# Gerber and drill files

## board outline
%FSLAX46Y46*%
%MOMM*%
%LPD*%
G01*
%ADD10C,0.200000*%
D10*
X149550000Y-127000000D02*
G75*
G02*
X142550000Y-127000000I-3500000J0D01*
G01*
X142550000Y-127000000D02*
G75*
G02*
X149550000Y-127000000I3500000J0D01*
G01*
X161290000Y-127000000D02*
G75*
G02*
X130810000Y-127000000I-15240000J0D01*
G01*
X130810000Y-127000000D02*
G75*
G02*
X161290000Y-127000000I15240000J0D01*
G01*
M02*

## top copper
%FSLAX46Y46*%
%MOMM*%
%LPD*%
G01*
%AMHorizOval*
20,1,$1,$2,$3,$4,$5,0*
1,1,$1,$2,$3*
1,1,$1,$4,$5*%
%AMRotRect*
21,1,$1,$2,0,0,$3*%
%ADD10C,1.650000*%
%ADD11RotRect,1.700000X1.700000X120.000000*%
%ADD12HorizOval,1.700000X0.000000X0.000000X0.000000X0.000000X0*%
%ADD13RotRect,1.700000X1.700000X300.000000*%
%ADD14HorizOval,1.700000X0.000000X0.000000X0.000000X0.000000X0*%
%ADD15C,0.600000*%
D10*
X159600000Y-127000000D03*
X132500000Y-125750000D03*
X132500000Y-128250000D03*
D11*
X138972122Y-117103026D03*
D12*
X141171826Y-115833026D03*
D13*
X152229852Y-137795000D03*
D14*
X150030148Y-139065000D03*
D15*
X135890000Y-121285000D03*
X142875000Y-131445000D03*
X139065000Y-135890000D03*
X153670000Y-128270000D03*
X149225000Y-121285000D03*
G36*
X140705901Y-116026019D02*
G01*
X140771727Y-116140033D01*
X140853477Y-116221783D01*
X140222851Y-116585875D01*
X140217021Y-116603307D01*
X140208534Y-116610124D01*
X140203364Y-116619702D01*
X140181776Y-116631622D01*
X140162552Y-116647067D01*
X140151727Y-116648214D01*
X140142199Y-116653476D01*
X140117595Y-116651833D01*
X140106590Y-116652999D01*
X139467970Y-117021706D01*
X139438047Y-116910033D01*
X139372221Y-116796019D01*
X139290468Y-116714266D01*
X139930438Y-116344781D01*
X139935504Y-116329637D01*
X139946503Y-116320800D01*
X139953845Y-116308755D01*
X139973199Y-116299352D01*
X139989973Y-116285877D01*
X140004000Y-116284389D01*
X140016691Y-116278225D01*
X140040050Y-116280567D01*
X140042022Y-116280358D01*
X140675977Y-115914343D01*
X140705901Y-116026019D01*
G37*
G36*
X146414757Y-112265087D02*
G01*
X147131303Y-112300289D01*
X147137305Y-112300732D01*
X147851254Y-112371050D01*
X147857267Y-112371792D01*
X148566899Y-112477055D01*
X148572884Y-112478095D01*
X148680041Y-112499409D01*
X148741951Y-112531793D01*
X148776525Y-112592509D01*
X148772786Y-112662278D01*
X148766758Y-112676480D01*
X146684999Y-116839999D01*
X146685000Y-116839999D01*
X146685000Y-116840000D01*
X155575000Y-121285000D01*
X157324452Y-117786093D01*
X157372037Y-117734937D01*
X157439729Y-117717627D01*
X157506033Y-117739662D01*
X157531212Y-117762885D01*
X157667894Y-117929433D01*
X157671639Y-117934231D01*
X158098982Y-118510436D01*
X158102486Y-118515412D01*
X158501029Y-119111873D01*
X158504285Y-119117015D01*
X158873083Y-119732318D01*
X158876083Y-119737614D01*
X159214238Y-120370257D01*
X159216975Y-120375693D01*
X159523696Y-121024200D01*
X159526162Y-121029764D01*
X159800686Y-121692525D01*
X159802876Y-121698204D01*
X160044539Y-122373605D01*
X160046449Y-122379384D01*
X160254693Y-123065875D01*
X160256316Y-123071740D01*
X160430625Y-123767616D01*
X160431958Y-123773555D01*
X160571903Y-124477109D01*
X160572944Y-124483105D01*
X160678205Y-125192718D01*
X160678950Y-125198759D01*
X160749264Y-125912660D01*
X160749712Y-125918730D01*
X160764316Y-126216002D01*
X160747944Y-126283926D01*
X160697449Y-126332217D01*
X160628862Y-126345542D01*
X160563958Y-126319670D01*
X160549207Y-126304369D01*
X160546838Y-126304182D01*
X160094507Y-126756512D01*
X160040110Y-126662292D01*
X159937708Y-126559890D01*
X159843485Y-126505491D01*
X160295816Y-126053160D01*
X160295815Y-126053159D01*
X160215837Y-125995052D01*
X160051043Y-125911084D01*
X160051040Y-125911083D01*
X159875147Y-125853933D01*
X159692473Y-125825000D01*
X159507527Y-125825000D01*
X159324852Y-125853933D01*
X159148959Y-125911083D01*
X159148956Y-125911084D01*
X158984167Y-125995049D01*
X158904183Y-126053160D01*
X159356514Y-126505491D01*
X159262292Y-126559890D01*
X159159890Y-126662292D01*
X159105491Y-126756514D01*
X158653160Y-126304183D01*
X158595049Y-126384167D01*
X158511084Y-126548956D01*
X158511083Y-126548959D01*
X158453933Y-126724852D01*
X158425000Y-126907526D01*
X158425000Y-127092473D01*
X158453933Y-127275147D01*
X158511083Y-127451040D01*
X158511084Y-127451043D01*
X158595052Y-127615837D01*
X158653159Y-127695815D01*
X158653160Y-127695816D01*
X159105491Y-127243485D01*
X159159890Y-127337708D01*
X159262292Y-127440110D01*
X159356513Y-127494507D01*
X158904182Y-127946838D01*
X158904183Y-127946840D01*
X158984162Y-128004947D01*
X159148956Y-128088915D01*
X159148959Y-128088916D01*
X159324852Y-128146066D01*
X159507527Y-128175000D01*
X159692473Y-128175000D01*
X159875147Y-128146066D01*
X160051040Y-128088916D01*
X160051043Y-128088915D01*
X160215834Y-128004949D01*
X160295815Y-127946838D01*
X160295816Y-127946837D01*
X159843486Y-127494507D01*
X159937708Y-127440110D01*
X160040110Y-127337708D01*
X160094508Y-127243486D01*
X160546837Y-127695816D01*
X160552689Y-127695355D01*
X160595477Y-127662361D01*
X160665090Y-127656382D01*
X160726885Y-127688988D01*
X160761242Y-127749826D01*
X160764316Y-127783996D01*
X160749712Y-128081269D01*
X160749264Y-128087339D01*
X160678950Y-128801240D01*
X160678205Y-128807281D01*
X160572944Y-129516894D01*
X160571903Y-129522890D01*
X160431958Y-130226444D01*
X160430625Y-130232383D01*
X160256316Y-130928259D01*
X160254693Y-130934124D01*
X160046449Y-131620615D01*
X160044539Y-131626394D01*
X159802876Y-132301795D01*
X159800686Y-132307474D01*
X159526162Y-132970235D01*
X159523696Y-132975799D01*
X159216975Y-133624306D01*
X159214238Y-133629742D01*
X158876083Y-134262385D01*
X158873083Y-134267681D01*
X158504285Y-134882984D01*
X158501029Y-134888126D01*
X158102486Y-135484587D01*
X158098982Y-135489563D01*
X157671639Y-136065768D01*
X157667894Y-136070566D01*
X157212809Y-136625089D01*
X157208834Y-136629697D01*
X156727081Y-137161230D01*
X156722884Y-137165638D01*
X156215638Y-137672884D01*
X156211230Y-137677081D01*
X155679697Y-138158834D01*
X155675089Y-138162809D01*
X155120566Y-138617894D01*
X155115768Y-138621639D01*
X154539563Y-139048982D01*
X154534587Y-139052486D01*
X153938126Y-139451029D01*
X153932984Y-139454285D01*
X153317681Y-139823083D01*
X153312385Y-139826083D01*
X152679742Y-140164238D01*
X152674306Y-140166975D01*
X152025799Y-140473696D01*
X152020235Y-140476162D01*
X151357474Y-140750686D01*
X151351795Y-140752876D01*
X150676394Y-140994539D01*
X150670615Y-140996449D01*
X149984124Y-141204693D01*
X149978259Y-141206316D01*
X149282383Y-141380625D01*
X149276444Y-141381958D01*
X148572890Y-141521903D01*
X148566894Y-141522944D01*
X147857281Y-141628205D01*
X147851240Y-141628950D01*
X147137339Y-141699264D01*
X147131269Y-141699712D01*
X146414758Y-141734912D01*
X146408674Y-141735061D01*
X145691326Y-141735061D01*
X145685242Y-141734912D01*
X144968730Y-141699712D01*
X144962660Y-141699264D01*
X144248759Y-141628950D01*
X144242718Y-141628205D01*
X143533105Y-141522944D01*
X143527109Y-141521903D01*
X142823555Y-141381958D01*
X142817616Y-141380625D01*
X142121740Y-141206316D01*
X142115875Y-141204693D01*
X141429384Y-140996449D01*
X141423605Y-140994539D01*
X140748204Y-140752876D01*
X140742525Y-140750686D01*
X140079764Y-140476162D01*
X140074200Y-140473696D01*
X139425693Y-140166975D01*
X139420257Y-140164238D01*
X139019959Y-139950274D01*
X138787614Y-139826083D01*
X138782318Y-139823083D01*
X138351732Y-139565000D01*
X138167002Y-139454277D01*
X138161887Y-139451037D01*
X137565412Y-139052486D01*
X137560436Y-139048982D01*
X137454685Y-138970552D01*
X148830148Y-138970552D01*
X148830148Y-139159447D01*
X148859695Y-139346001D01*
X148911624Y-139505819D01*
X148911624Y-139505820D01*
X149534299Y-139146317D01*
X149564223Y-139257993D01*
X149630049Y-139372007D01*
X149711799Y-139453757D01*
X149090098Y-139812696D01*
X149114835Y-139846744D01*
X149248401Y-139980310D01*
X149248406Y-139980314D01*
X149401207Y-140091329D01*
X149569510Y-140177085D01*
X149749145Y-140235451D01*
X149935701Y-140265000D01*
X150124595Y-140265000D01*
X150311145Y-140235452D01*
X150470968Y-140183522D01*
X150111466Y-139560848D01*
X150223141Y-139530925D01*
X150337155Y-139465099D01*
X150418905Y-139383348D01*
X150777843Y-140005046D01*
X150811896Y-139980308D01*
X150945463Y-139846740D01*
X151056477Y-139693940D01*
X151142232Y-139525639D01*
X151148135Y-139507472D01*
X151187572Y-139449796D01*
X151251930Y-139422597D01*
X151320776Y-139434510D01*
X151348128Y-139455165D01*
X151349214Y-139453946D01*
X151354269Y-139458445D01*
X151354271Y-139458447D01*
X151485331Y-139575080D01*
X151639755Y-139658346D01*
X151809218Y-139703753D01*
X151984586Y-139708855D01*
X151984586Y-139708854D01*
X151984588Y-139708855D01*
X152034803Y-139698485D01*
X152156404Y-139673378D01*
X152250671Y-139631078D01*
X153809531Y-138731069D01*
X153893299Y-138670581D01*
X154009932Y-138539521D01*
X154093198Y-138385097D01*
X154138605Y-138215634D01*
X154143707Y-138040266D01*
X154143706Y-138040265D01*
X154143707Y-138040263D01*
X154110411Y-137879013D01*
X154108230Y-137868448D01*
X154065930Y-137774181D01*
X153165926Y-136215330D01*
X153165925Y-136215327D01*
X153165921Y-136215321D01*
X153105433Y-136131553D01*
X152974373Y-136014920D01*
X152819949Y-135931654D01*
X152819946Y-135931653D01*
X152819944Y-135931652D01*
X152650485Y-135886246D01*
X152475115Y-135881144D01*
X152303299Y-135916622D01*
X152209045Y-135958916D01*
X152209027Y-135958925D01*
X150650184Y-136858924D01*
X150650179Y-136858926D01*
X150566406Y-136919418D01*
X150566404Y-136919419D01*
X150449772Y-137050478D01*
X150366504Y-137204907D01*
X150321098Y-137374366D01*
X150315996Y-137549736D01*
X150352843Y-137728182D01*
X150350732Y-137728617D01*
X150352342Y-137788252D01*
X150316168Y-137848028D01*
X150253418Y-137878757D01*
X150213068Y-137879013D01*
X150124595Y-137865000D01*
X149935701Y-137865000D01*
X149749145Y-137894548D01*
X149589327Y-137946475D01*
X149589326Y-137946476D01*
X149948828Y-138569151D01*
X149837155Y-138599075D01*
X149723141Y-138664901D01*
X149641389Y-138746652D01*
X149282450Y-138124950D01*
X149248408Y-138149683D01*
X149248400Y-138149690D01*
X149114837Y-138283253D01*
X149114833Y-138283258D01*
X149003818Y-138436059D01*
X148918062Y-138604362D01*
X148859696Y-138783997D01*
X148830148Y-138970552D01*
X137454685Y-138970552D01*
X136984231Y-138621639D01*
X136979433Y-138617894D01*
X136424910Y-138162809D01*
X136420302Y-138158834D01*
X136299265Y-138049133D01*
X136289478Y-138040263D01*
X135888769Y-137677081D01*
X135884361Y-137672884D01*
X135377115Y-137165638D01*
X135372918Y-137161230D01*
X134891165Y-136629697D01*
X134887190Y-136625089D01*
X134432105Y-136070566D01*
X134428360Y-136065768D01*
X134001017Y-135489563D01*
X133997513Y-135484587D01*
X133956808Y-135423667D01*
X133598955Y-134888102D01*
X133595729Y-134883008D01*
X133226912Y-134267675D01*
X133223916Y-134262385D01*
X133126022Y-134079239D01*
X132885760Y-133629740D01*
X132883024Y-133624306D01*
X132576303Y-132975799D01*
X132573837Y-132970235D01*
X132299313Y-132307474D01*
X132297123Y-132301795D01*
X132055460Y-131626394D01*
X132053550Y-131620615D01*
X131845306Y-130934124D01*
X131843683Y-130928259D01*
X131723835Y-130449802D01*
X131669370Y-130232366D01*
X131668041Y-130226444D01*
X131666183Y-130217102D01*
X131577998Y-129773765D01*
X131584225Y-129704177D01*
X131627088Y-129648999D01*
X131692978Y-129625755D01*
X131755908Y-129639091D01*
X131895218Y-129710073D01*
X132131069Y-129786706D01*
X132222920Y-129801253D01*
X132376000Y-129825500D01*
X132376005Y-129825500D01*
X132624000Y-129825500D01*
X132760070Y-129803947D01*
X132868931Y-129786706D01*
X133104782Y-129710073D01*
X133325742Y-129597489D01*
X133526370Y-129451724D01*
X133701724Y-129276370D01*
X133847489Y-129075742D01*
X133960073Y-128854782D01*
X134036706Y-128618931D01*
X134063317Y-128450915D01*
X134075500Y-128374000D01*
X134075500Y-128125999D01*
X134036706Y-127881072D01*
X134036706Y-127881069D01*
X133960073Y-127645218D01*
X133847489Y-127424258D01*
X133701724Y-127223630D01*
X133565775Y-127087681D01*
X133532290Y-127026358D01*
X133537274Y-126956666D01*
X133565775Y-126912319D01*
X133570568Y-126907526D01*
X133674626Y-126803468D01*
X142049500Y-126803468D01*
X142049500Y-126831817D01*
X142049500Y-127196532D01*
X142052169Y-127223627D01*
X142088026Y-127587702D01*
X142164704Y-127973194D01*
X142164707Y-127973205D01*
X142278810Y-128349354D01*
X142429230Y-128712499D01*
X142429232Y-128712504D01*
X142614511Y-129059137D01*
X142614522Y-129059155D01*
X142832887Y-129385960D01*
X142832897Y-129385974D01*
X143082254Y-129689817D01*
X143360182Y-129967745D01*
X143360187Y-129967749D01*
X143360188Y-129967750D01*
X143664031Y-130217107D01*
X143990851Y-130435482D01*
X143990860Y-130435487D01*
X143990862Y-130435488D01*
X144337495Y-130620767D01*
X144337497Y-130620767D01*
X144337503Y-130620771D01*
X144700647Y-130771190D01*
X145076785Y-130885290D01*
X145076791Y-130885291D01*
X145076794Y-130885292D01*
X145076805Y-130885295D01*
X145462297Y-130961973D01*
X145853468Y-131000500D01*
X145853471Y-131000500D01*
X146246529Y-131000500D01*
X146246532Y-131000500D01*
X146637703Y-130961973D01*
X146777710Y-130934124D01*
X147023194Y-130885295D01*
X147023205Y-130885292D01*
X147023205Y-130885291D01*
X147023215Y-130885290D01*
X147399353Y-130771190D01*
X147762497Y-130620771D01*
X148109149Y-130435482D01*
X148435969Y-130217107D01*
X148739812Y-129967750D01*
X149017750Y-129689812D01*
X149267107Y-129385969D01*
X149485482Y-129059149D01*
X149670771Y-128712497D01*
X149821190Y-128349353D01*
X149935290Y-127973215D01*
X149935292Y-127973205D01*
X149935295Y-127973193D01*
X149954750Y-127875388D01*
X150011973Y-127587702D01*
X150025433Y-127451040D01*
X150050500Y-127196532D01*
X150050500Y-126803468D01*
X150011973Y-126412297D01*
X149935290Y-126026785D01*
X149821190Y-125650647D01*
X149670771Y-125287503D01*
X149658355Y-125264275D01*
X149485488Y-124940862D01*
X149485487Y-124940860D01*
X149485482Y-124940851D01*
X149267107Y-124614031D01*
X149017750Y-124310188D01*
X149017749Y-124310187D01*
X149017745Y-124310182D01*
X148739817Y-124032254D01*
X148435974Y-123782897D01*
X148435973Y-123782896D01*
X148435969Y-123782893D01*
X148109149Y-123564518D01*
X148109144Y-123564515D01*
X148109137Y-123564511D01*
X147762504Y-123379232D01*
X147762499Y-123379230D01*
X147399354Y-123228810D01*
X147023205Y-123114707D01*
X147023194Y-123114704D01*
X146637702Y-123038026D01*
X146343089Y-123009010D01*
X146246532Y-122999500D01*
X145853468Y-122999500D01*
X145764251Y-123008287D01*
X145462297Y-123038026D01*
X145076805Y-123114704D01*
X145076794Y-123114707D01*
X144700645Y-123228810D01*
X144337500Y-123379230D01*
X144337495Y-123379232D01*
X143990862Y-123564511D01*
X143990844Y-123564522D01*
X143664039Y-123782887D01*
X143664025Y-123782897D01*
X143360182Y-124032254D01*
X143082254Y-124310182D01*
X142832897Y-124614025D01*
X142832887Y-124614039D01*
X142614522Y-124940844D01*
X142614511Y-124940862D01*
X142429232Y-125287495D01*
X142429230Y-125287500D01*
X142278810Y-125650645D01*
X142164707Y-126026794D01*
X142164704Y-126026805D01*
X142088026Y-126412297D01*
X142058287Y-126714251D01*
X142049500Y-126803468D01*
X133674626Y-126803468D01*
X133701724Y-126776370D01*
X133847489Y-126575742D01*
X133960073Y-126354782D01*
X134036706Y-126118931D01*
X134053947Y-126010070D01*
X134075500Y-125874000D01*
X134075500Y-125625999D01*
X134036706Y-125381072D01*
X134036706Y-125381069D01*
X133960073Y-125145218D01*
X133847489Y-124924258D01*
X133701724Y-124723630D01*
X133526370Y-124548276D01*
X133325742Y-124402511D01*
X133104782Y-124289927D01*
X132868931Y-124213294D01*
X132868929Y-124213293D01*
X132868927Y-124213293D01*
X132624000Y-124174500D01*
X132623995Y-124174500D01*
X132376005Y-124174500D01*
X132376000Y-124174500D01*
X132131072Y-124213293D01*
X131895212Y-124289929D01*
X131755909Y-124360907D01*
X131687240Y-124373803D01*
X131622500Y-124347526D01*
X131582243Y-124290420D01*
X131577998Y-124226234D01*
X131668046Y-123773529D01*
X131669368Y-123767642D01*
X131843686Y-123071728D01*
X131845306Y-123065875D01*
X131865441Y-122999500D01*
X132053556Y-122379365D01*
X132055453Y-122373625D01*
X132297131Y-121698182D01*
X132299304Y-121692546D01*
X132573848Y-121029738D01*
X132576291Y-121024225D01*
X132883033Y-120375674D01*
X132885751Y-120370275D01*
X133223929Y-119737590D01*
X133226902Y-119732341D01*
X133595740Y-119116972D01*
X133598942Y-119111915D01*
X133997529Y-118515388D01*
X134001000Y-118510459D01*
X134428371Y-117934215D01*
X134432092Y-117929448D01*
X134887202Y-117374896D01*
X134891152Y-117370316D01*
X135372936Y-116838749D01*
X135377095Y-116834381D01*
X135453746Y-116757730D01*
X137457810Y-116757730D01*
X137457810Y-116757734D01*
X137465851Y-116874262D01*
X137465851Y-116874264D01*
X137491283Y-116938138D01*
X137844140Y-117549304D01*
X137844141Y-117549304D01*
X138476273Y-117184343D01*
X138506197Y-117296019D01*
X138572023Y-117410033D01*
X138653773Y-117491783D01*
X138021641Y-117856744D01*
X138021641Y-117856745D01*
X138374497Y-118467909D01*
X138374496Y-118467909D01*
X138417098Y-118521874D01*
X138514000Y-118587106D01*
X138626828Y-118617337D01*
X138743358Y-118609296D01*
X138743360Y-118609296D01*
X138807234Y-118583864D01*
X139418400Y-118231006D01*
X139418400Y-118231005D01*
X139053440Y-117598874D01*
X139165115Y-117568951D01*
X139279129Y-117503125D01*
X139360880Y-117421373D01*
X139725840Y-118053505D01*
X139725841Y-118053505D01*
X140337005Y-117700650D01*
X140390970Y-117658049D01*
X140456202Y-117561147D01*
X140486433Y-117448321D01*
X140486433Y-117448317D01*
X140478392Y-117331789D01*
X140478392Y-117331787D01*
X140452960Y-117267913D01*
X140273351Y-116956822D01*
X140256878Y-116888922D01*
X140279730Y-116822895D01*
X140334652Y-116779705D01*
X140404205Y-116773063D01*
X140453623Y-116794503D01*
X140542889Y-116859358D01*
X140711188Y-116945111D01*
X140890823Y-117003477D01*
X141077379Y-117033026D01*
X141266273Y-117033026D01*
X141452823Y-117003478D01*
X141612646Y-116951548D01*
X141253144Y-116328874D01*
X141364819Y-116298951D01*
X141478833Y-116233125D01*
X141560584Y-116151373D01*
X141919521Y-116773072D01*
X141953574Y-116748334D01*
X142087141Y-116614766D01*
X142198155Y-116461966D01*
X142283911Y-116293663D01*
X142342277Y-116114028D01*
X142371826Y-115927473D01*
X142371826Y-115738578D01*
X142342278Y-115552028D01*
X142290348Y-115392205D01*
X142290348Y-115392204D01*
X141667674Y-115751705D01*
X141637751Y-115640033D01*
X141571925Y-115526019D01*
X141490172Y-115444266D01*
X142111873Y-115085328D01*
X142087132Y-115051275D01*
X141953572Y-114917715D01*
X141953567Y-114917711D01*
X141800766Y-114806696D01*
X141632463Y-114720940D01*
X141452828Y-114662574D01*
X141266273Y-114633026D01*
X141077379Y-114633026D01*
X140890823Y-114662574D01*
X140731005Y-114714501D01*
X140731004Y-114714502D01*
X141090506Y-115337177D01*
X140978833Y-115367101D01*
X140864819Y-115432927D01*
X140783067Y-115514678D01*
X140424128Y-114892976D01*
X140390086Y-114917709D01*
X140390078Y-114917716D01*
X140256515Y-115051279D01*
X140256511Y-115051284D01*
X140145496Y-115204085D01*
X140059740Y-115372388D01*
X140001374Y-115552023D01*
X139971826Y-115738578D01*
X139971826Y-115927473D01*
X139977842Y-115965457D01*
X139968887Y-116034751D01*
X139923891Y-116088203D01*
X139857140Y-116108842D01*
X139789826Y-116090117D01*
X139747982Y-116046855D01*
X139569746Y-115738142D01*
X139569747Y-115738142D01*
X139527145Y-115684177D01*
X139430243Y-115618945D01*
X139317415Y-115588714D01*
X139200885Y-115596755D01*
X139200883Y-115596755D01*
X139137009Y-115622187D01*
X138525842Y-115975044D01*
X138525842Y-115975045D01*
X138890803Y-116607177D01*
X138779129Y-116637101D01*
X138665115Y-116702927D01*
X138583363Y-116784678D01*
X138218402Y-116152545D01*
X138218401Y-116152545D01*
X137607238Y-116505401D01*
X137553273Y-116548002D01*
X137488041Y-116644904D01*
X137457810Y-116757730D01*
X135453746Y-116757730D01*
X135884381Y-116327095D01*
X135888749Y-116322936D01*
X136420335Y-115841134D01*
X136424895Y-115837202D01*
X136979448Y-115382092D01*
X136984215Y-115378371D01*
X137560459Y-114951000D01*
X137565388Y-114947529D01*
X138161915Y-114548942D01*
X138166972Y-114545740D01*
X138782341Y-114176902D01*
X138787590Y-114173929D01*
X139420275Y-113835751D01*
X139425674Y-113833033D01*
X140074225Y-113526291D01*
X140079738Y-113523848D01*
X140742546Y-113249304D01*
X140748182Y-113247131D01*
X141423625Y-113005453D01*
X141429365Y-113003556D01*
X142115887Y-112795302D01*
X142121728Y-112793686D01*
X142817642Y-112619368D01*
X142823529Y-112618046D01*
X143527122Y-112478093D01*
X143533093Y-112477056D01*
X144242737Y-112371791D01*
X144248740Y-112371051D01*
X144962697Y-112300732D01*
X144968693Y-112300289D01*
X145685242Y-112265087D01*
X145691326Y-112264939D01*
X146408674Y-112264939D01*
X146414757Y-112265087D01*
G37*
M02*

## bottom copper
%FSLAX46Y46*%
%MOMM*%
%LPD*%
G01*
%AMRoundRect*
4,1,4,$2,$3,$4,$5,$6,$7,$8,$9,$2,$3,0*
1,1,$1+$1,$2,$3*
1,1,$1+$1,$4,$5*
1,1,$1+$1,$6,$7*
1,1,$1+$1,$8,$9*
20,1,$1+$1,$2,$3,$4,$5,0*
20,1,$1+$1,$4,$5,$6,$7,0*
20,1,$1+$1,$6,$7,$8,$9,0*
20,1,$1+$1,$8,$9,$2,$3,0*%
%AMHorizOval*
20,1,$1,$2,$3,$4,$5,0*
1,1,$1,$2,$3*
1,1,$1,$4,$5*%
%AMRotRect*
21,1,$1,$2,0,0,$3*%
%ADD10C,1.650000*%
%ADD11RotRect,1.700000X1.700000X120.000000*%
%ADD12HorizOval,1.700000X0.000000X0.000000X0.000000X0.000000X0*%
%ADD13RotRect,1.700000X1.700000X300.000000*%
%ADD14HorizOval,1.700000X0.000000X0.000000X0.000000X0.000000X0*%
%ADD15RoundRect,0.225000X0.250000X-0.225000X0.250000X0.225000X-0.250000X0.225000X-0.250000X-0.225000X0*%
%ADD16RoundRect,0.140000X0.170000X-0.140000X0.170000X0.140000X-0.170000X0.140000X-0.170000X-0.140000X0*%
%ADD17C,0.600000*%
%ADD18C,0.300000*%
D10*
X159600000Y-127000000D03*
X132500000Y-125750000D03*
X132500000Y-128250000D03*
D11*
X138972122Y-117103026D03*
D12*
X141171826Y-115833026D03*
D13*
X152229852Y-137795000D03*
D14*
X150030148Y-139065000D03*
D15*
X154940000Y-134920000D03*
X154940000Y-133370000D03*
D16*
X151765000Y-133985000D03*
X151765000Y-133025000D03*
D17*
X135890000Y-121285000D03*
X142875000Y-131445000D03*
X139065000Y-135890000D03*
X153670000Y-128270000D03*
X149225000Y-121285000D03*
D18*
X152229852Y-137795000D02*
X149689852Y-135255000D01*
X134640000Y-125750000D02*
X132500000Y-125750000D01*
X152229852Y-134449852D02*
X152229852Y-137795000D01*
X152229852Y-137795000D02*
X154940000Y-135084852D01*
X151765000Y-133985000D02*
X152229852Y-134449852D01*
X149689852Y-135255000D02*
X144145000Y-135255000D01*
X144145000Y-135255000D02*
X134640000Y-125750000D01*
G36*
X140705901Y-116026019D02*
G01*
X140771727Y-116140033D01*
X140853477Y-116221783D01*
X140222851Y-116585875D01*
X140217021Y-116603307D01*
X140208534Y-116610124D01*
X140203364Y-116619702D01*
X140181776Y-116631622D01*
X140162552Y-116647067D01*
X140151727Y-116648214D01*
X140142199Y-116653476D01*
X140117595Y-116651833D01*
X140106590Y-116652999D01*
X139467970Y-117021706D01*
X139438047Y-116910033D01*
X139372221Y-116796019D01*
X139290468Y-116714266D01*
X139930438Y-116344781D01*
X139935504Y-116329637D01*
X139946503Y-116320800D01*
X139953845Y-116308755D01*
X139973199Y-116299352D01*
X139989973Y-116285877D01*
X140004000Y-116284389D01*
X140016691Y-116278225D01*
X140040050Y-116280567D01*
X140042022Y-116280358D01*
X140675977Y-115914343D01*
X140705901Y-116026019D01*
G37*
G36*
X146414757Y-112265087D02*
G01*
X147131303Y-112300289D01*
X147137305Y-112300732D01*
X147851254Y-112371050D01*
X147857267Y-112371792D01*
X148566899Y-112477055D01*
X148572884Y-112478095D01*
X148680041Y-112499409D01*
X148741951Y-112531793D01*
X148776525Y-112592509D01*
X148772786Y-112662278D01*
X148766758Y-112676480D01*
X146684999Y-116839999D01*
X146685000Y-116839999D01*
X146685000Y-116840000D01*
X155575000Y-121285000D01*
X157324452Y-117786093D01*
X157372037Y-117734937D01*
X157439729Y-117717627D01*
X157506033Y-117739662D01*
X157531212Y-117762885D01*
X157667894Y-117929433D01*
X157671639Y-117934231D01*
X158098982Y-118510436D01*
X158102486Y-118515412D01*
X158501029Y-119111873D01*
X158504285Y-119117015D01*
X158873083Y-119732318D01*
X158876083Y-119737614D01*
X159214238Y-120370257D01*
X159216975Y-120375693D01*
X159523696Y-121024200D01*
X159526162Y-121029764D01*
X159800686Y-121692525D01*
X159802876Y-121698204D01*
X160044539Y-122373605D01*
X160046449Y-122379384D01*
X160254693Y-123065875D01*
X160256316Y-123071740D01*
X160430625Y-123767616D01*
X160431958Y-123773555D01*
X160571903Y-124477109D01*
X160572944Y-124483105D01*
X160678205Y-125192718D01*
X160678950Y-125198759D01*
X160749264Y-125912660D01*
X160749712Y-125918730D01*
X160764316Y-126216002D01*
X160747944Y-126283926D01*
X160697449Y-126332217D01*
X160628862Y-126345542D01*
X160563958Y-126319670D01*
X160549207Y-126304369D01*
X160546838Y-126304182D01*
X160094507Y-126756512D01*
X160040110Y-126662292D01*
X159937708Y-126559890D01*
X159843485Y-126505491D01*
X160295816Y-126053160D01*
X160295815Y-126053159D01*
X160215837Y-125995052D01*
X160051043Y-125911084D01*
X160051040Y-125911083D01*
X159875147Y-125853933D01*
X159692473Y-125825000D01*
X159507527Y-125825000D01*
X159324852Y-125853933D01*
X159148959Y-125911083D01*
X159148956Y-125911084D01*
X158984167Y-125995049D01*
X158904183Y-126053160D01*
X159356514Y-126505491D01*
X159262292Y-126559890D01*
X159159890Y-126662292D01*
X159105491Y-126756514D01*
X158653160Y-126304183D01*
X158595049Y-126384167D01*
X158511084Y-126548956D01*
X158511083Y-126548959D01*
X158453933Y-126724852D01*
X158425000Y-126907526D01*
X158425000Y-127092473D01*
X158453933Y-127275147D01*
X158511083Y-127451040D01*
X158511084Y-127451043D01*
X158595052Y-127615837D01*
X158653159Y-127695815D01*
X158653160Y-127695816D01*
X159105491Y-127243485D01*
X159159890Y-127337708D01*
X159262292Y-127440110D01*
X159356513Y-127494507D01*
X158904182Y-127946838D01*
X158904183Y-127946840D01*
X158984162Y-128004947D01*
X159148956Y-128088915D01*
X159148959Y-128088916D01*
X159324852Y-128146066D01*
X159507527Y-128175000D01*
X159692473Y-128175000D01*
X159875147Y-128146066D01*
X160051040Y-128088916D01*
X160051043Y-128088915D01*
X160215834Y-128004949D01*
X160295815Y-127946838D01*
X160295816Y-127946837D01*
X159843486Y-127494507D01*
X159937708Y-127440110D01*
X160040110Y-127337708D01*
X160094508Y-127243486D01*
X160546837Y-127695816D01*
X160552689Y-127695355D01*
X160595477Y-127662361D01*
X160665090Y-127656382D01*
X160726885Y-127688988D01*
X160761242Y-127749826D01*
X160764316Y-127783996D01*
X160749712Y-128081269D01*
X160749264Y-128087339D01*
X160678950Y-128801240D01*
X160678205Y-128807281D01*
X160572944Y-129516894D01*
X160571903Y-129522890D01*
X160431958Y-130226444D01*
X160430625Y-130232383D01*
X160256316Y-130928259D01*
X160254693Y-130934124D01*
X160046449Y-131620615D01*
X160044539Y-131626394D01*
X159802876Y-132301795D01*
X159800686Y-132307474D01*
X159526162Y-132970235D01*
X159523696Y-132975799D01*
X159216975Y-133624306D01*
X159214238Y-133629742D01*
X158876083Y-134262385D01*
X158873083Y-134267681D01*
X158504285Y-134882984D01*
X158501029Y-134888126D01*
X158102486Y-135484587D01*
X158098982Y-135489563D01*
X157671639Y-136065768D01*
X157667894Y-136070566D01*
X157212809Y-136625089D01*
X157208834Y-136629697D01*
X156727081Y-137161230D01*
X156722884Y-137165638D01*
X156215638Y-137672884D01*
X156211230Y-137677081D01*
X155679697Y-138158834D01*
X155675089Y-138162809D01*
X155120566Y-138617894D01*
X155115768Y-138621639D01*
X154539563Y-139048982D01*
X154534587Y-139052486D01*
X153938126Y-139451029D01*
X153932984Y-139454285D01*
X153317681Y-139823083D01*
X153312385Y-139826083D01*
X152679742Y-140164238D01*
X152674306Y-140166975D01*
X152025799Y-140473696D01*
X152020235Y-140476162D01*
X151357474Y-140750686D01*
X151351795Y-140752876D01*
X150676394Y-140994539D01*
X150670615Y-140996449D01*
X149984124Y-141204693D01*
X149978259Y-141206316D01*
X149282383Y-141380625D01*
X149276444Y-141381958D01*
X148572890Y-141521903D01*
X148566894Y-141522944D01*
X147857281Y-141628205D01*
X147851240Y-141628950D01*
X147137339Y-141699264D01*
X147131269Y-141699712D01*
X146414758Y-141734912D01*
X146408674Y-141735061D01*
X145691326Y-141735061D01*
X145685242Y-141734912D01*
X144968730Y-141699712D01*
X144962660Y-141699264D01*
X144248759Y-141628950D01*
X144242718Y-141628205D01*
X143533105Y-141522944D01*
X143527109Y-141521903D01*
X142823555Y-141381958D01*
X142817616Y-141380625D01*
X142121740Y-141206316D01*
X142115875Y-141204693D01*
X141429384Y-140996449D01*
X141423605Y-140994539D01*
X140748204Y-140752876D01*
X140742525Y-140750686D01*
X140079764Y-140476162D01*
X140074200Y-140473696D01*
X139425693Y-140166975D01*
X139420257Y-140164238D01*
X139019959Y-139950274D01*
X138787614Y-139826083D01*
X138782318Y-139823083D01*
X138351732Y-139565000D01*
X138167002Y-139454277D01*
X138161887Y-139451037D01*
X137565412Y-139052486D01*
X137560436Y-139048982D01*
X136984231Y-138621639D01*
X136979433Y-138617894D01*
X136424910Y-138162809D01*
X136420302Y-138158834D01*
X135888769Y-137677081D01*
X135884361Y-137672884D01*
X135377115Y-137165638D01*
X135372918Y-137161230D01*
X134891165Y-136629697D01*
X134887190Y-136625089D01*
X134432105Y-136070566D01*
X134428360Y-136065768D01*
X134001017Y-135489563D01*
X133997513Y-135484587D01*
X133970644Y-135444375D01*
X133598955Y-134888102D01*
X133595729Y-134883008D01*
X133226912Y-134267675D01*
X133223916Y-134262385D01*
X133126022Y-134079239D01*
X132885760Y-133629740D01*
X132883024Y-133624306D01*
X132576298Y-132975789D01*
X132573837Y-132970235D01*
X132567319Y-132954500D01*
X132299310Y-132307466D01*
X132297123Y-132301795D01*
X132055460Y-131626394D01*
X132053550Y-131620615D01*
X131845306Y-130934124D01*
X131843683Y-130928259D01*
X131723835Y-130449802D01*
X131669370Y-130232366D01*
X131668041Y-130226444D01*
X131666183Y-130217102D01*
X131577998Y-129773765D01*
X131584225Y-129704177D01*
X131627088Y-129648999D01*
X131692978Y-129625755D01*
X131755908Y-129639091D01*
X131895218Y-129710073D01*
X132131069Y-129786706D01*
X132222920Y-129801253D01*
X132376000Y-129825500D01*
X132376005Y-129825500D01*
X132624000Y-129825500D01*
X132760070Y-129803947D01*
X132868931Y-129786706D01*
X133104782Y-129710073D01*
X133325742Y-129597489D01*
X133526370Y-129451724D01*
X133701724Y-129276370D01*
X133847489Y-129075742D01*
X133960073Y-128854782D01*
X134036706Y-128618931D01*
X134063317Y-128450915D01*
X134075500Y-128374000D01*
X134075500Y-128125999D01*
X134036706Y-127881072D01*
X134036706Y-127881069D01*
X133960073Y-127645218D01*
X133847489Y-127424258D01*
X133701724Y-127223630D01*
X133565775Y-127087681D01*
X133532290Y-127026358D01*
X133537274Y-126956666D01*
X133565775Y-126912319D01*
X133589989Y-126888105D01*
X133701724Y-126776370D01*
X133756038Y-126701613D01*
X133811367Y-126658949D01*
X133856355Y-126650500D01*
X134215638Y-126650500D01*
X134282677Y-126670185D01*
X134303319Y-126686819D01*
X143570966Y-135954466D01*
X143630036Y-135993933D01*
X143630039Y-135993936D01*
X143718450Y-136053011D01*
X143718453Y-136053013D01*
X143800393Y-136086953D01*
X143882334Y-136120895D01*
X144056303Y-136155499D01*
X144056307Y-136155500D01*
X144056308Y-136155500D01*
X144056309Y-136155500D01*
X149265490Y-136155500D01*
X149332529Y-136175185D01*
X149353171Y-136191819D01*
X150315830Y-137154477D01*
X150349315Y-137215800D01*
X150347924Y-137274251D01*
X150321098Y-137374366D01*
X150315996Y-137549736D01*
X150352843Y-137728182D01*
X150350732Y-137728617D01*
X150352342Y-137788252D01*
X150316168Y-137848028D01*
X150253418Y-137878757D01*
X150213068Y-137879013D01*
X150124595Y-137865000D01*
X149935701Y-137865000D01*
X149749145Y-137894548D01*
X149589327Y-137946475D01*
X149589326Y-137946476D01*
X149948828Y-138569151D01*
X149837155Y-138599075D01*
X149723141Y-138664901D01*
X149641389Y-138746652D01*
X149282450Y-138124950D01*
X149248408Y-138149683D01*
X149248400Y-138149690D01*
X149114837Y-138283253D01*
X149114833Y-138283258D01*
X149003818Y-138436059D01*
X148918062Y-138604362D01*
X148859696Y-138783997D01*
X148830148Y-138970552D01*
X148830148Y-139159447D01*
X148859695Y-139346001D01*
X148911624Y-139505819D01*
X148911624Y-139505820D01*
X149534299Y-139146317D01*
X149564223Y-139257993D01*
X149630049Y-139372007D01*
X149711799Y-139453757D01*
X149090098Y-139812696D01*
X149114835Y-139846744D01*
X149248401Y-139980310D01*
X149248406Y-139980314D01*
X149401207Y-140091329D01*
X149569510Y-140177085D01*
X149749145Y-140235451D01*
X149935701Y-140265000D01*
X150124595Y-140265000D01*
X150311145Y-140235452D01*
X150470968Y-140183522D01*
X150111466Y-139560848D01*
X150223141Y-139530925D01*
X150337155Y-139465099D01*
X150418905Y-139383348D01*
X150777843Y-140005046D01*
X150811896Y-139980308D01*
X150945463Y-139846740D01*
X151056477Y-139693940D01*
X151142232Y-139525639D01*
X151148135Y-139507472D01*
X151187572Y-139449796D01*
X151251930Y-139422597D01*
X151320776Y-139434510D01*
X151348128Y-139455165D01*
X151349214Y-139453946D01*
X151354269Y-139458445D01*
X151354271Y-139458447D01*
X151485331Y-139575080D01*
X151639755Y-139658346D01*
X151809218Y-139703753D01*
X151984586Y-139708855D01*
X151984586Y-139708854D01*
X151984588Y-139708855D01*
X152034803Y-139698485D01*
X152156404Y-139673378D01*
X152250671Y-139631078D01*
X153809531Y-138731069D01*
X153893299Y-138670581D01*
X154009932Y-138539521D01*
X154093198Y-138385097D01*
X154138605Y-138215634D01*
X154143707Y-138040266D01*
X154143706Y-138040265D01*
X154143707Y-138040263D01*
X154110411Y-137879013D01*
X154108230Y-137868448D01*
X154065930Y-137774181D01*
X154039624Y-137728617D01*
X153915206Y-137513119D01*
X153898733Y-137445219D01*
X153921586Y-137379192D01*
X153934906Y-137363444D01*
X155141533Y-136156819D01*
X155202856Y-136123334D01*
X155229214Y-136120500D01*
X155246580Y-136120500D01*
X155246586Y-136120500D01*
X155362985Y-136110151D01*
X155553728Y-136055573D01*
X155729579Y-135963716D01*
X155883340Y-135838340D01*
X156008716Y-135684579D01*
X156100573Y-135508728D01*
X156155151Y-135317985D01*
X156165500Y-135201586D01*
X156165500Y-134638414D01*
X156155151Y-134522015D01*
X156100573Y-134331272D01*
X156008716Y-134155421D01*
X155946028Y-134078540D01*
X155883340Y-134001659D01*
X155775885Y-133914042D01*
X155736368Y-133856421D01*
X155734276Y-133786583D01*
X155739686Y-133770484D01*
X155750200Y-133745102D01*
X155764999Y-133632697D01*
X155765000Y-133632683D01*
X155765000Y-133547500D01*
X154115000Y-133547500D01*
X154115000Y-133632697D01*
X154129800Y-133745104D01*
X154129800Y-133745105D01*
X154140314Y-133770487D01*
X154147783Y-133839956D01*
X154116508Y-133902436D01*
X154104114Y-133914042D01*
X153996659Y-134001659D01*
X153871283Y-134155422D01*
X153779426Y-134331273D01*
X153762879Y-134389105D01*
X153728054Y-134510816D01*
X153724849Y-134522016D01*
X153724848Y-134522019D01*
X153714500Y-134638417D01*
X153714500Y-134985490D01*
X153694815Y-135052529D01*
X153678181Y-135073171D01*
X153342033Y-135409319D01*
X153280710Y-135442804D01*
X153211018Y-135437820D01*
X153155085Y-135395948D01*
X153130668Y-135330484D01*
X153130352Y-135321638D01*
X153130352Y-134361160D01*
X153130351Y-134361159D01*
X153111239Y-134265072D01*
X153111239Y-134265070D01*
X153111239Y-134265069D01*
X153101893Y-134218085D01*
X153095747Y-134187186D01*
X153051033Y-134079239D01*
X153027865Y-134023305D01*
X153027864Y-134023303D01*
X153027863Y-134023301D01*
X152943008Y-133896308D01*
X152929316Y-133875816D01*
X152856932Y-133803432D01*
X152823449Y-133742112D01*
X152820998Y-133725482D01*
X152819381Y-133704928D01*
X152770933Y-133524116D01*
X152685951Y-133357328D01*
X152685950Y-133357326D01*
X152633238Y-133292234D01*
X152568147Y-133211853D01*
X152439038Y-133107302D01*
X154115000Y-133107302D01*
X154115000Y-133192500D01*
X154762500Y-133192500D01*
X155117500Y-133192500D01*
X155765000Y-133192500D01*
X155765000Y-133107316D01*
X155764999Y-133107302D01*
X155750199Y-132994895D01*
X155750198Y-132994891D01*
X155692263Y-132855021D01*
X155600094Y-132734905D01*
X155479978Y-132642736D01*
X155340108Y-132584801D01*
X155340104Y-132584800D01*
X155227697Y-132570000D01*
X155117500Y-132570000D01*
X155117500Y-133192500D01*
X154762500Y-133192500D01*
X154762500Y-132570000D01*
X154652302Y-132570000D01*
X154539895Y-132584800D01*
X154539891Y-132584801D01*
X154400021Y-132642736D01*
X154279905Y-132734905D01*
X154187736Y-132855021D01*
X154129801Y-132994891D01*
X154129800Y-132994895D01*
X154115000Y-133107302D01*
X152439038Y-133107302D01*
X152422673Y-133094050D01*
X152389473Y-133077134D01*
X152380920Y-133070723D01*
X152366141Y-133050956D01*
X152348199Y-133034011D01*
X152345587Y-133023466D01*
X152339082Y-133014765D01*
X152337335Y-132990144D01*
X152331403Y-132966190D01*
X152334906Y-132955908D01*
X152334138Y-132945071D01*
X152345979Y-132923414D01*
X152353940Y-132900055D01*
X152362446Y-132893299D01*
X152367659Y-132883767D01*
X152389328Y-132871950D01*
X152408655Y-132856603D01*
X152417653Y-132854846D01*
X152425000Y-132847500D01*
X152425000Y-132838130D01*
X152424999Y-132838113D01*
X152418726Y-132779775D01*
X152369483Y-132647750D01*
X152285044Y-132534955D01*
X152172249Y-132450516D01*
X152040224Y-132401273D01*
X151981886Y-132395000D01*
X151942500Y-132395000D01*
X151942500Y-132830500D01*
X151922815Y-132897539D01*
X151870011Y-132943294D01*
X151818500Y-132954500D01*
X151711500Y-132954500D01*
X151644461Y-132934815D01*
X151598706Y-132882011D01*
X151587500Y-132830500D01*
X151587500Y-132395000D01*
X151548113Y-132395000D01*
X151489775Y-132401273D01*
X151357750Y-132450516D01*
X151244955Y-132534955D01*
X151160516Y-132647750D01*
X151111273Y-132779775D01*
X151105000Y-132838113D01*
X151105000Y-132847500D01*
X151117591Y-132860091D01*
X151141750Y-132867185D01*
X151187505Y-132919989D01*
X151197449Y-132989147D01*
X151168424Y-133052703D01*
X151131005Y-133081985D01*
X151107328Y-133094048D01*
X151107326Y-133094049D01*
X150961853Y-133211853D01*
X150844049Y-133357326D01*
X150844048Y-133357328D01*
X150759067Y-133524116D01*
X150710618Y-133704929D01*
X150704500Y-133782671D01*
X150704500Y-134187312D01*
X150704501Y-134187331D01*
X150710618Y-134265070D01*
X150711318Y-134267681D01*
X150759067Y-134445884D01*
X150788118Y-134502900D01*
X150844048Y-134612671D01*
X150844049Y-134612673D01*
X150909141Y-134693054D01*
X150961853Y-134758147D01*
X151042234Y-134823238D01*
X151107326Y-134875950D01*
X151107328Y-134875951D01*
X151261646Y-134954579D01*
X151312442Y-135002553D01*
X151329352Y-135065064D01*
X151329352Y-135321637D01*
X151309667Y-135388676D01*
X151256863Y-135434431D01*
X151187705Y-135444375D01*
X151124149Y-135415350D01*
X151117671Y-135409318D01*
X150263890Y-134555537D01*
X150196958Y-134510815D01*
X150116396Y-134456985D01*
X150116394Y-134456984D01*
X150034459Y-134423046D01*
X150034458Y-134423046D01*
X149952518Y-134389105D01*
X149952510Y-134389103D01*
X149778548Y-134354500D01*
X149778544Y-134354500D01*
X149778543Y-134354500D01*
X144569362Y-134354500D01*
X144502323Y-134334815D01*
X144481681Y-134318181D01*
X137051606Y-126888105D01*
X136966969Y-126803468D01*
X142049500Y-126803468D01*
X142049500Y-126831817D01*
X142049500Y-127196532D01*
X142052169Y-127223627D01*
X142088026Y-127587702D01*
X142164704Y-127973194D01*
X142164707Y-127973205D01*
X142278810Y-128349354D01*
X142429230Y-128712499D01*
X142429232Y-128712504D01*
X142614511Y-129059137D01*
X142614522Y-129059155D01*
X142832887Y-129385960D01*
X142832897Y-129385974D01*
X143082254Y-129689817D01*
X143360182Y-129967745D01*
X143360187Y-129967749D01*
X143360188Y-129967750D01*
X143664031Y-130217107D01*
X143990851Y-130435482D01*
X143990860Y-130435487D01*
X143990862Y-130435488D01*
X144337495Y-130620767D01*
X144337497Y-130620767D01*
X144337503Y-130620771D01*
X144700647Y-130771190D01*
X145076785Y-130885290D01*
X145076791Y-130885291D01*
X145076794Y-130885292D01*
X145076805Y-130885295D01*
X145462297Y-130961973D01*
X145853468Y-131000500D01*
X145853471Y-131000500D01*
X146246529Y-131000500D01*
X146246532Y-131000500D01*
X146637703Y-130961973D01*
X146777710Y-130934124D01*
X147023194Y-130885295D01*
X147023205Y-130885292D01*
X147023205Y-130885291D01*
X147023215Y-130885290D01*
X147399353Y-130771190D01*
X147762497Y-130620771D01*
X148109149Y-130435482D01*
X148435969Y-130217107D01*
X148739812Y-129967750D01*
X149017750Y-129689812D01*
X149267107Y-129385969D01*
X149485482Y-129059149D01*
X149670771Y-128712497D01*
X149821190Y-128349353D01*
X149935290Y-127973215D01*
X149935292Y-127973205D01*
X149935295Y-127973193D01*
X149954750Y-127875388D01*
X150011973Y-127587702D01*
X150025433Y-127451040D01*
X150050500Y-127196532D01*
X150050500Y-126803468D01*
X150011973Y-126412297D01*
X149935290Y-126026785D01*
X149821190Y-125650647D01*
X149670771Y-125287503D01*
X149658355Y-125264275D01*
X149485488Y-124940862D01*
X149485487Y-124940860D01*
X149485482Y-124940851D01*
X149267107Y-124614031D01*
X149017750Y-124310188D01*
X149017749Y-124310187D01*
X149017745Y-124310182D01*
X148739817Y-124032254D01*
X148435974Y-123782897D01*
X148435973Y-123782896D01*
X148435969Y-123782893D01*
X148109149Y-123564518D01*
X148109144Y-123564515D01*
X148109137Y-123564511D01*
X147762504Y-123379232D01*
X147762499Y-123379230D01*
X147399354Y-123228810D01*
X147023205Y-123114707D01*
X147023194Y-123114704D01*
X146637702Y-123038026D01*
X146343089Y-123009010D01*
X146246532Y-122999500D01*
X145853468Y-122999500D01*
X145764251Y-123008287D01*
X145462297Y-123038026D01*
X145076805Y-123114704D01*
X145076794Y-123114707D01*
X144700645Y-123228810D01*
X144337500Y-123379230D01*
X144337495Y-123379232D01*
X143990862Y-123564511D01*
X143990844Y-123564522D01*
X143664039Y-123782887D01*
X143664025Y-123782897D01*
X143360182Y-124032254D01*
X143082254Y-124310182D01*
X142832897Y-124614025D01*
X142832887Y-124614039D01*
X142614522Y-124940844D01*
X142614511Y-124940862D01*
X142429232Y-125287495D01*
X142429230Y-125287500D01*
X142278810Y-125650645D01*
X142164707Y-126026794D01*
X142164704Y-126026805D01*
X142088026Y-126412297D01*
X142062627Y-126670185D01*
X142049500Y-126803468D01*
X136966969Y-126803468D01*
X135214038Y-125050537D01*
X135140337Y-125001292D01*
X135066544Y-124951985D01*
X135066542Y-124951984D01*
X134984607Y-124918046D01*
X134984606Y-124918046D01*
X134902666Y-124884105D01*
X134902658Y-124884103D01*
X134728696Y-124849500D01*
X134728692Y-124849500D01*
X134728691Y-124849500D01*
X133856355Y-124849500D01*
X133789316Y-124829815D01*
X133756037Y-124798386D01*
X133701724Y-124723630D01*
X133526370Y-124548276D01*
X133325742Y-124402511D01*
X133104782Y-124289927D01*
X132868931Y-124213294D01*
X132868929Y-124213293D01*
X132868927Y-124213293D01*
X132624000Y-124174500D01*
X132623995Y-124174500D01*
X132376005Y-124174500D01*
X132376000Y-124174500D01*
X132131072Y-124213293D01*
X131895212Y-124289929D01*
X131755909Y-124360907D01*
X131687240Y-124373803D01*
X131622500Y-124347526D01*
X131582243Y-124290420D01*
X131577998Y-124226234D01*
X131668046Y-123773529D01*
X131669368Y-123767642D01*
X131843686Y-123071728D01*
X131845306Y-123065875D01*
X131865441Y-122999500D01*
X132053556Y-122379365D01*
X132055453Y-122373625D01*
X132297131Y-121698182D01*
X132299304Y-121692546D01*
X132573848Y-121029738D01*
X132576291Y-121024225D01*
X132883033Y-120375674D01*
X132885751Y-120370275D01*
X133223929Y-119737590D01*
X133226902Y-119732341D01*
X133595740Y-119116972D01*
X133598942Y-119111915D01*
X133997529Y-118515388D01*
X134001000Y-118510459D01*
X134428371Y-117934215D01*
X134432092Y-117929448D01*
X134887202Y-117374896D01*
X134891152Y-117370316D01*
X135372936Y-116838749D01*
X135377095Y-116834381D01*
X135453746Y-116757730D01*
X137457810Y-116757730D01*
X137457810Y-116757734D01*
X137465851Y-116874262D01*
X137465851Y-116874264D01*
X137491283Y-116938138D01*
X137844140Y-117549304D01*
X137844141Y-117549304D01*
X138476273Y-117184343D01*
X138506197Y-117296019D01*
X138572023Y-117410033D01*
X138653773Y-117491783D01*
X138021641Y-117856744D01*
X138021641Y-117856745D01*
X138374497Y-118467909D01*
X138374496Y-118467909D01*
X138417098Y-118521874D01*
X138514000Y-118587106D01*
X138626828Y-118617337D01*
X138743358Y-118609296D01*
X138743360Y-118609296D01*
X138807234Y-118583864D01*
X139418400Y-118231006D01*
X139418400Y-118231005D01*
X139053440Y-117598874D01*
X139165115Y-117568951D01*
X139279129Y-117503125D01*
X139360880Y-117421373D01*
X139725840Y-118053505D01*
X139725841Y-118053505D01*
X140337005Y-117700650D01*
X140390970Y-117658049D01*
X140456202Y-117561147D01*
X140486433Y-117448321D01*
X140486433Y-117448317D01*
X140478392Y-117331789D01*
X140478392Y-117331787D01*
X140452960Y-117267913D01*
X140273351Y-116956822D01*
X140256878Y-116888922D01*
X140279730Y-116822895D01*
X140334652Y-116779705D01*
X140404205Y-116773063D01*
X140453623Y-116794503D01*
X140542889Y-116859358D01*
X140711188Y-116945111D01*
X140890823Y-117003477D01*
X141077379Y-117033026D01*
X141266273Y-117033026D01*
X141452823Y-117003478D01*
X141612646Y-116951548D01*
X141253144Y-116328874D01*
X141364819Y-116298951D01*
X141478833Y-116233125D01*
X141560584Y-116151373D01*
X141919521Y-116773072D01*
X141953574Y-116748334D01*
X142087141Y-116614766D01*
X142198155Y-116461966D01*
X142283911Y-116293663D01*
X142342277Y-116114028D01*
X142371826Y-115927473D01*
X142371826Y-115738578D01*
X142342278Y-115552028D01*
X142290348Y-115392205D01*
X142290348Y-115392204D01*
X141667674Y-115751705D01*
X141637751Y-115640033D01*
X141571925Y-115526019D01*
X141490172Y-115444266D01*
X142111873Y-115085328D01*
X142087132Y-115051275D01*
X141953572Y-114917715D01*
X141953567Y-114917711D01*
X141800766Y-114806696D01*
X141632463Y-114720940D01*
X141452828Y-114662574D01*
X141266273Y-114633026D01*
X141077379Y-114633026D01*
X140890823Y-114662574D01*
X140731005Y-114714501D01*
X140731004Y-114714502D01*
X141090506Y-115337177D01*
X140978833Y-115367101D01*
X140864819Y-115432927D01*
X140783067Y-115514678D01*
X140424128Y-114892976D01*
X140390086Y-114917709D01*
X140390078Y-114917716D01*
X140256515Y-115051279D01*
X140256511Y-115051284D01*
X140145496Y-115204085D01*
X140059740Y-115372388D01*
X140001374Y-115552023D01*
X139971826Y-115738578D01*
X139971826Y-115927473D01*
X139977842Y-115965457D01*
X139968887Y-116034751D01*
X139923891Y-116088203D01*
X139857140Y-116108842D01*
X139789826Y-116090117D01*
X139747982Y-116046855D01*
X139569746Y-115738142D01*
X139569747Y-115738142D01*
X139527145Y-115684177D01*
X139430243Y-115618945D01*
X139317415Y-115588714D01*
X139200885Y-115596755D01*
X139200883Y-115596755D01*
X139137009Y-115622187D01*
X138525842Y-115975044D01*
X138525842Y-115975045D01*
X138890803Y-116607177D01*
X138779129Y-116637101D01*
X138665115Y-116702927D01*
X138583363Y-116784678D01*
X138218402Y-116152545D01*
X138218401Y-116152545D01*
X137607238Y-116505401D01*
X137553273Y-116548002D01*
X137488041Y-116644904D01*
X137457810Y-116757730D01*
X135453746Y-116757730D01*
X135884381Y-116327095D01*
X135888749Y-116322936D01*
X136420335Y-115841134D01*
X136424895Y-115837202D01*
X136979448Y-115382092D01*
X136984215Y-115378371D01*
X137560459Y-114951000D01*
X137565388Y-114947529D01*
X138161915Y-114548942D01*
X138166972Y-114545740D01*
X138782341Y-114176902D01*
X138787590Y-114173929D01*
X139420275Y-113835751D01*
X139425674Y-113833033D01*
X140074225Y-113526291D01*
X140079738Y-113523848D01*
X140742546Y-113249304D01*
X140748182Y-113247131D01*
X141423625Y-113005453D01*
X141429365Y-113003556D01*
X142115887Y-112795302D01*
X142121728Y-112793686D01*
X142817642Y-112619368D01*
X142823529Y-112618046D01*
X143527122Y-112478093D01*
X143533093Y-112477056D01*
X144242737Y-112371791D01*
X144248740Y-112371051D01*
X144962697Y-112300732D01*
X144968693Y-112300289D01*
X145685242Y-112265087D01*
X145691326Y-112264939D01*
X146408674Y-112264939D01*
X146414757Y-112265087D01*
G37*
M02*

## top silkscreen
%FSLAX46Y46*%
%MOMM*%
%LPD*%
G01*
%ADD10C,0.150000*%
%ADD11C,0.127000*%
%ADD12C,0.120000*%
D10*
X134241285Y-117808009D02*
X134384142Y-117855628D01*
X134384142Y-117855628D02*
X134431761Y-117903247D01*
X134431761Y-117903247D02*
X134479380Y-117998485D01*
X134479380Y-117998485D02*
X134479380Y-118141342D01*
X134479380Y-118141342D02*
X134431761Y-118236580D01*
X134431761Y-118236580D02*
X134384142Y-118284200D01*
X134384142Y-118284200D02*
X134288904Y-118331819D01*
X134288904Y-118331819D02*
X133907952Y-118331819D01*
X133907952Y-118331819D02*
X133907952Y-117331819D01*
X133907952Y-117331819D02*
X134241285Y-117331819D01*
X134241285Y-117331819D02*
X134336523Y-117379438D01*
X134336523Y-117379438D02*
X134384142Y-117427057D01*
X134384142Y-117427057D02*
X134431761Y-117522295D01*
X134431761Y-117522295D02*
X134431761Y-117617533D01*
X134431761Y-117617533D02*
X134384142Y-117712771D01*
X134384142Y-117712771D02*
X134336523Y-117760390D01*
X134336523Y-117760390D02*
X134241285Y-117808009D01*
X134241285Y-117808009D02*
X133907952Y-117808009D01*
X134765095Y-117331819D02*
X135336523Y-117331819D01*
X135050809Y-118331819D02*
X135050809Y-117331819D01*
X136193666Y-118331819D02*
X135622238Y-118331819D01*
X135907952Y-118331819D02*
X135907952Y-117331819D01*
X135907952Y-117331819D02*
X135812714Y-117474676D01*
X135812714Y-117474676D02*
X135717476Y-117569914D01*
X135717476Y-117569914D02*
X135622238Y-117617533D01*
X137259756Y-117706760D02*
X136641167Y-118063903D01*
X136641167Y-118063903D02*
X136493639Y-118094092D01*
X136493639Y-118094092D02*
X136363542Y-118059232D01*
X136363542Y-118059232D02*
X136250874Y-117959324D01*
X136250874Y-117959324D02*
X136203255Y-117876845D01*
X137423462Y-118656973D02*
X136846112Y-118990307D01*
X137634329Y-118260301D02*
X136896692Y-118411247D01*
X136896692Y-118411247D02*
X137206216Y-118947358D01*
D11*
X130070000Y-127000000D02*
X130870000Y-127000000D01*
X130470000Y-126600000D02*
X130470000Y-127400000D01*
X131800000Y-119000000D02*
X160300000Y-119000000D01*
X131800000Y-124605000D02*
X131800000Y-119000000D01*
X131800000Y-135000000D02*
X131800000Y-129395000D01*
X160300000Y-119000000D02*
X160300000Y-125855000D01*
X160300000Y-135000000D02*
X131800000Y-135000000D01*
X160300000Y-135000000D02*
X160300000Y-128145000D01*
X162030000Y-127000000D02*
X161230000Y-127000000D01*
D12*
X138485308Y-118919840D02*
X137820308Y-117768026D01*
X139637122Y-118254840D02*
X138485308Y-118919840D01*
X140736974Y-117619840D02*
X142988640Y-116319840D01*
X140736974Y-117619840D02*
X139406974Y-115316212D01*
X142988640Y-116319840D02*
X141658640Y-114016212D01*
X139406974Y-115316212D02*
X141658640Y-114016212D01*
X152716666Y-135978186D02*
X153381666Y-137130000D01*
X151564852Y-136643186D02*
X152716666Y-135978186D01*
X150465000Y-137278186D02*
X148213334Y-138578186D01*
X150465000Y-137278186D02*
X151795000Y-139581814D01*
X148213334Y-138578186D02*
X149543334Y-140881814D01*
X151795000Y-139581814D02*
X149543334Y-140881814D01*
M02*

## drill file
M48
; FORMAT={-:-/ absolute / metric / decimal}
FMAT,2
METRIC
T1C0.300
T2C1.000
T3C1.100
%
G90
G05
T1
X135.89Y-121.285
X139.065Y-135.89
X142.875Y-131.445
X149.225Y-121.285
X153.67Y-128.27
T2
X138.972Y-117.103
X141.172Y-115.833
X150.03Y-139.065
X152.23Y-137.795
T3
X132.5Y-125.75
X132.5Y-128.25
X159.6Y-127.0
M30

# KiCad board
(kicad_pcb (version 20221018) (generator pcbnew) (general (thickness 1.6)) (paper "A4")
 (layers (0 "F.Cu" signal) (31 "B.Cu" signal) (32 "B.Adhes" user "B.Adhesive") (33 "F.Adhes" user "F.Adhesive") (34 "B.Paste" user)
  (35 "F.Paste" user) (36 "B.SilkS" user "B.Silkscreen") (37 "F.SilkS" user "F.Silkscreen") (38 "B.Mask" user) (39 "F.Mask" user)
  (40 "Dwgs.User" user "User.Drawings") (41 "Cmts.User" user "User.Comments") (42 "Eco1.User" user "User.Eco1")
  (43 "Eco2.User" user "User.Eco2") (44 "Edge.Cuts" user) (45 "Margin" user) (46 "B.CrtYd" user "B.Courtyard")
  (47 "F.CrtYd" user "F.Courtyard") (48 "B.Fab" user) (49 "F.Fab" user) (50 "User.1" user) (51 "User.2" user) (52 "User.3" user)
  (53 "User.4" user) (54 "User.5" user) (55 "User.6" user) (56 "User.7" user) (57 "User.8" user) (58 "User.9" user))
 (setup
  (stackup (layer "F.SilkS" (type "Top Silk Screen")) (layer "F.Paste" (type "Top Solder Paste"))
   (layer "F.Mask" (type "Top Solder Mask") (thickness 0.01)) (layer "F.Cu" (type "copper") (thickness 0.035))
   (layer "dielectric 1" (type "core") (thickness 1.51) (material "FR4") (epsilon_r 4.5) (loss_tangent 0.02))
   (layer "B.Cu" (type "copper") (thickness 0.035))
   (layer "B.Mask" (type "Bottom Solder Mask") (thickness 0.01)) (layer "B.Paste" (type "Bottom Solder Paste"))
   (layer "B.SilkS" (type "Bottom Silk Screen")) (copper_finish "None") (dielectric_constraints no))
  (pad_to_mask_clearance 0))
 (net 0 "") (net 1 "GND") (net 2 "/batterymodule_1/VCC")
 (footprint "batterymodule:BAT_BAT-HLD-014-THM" (layer "F.Cu") (at 146.05 127)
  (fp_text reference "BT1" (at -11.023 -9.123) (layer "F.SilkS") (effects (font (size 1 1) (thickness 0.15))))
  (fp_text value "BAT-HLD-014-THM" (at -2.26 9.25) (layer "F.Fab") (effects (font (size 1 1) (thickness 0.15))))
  (fp_line (start -15.98 0) (end -15.18 0) (stroke (width 0.127) (type solid)) (layer "F.SilkS"))
  (fp_line (start -15.58 -0.4) (end -15.58 0.4) (stroke (width 0.127) (type solid)) (layer "F.SilkS"))
  (fp_line (start -14.25 -8) (end 14.25 -8) (stroke (width 0.127) (type solid)) (layer "F.SilkS"))
  (fp_line (start -14.25 -2.395) (end -14.25 -8) (stroke (width 0.127) (type solid)) (layer "F.SilkS"))
  (fp_line (start -14.25 8) (end -14.25 2.395) (stroke (width 0.127) (type solid)) (layer "F.SilkS"))
  (fp_line (start 14.25 -8) (end 14.25 -1.145) (stroke (width 0.127) (type solid)) (layer "F.SilkS"))
  (fp_line (start 14.25 8) (end -14.25 8) (stroke (width 0.127) (type solid)) (layer "F.SilkS"))
  (fp_line (start 14.25 8) (end 14.25 1.145) (stroke (width 0.127) (type solid)) (layer "F.SilkS"))
  (fp_line (start 15.98 0) (end 15.18 0) (stroke (width 0.127) (type solid)) (layer "F.SilkS"))
  (pad "N" thru_hole circle (at 13.55 0) (size 1.65 1.65) (drill 1.1) (layers "*.Cu" "*.Mask") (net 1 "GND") (solder_mask_margin 0.102))
  (pad "P_1" thru_hole circle (at -13.55 -1.25) (size 1.65 1.65) (drill 1.1) (layers "*.Cu" "*.Mask") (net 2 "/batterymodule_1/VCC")
   (solder_mask_margin 0.102))
  (pad "P_2" thru_hole circle (at -13.55 1.25) (size 1.65 1.65) (drill 1.1) (layers "*.Cu" "*.Mask") (solder_mask_margin 0.102)))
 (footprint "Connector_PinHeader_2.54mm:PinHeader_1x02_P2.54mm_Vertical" (layer "F.Cu") (at 140.071974 116.468026 120)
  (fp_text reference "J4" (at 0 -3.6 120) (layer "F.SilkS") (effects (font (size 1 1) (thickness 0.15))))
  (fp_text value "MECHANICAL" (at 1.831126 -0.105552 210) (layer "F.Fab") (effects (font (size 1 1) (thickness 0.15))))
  (fp_line (start -1.33 -2.6) (end 0 -2.6) (stroke (width 0.12) (type solid)) (layer "F.SilkS"))
  (fp_line (start -1.33 -1.27) (end -1.33 -2.6) (stroke (width 0.12) (type solid)) (layer "F.SilkS"))
  (fp_line (start -1.33 0) (end -1.33 2.6) (stroke (width 0.12) (type solid)) (layer "F.SilkS"))
  (fp_line (start -1.33 0) (end 1.33 0) (stroke (width 0.12) (type solid)) (layer "F.SilkS"))
  (fp_line (start -1.33 2.6) (end 1.33 2.6) (stroke (width 0.12) (type solid)) (layer "F.SilkS"))
  (fp_line (start 1.33 0) (end 1.33 2.6) (stroke (width 0.12) (type solid)) (layer "F.SilkS"))
  (pad "1" thru_hole rect (at 0 -1.27 120) (size 1.7 1.7) (drill 1) (layers "*.Cu" "*.Mask") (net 1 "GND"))
  (pad "2" thru_hole oval (at 0 1.27 120) (size 1.7 1.7) (drill 1) (layers "*.Cu" "*.Mask") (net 1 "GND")))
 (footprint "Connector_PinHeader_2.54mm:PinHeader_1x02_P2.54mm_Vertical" (layer "F.Cu") (at 151.13 138.43 -60)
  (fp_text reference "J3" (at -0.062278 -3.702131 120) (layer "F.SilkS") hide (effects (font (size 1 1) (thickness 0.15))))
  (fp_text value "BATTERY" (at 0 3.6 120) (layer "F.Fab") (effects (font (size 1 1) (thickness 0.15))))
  (fp_line (start -1.33 -2.6) (end 0 -2.6) (stroke (width 0.12) (type solid)) (layer "F.SilkS"))
  (fp_line (start -1.33 -1.27) (end -1.33 -2.6) (stroke (width 0.12) (type solid)) (layer "F.SilkS"))
  (fp_line (start -1.33 0) (end -1.33 2.6) (stroke (width 0.12) (type solid)) (layer "F.SilkS"))
  (fp_line (start -1.33 0) (end 1.33 0) (stroke (width 0.12) (type solid)) (layer "F.SilkS"))
  (fp_line (start -1.33 2.6) (end 1.33 2.6) (stroke (width 0.12) (type solid)) (layer "F.SilkS"))
  (fp_line (start 1.33 0) (end 1.33 2.6) (stroke (width 0.12) (type solid)) (layer "F.SilkS"))
  (pad "1" thru_hole rect (at 0 -1.27 300) (size 1.7 1.7) (drill 1) (layers "*.Cu" "*.Mask") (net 2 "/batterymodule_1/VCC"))
  (pad "2" thru_hole oval (at 0 1.27 300) (size 1.7 1.7) (drill 1) (layers "*.Cu" "*.Mask") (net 1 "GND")))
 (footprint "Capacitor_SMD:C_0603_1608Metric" (layer "B.Cu") (at 154.94 134.145 90)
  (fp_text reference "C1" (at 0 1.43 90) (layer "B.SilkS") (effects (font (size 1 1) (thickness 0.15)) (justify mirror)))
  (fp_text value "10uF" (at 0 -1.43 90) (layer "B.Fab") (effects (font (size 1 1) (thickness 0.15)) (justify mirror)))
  (pad "1" smd roundrect (at -0.775 0 90) (size 0.9 0.95) (layers "B.Cu" "B.Paste" "B.Mask") (roundrect_rratio 0.25)
   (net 2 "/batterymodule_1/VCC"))
  (pad "2" smd roundrect (at 0.775 0 90) (size 0.9 0.95) (layers "B.Cu" "B.Paste" "B.Mask") (roundrect_rratio 0.25) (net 1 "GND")))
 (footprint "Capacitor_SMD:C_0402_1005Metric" (layer "B.Cu") (at 151.765 133.505 90)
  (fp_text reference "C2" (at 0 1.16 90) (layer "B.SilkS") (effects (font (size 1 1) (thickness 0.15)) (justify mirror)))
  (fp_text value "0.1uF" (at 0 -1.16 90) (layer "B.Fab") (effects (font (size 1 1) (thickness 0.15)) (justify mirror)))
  (pad "1" smd roundrect (at -0.48 0 90) (size 0.56 0.62) (layers "B.Cu" "B.Paste" "B.Mask") (roundrect_rratio 0.25)
   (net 2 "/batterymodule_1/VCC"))
  (pad "2" smd roundrect (at 0.48 0 90) (size 0.56 0.62) (layers "B.Cu" "B.Paste" "B.Mask") (roundrect_rratio 0.25) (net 1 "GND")))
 (gr_circle (center 146.05 127) (end 149.55 127) (stroke (width 0.2) (type default)) (fill none) (layer "Edge.Cuts"))
 (gr_circle (center 146.05 127) (end 161.29 127) (stroke (width 0.2) (type default)) (fill none) (layer "Edge.Cuts"))
 (segment (start 152.229852 137.795) (end 149.689852 135.255) (width 0.3) (layer "B.Cu") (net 2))
 (segment (start 134.64 125.75) (end 132.5 125.75) (width 0.3) (layer "B.Cu") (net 2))
 (segment (start 152.229852 134.449852) (end 152.229852 137.795) (width 0.3) (layer "B.Cu") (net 2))
 (segment (start 152.229852 137.795) (end 154.94 135.084852) (width 0.3) (layer "B.Cu") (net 2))
 (segment (start 151.765 133.985) (end 152.229852 134.449852) (width 0.3) (layer "B.Cu") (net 2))
 (segment (start 149.689852 135.255) (end 144.145 135.255) (width 0.3) (layer "B.Cu") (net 2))
 (segment (start 144.145 135.255) (end 134.64 125.75) (width 0.3) (layer "B.Cu") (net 2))
 (via (at 135.89 121.285) (size 0.6) (drill 0.3) (layers "F.Cu" "B.Cu") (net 1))
 (via (at 142.875 131.445) (size 0.6) (drill 0.3) (layers "F.Cu" "B.Cu") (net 1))
 (via (at 139.065 135.89) (size 0.6) (drill 0.3) (layers "F.Cu" "B.Cu") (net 1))
 (via (at 153.67 128.27) (size 0.6) (drill 0.3) (layers "F.Cu" "B.Cu") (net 1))
 (via (at 149.225 121.285) (size 0.6) (drill 0.3) (layers "F.Cu" "B.Cu") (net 1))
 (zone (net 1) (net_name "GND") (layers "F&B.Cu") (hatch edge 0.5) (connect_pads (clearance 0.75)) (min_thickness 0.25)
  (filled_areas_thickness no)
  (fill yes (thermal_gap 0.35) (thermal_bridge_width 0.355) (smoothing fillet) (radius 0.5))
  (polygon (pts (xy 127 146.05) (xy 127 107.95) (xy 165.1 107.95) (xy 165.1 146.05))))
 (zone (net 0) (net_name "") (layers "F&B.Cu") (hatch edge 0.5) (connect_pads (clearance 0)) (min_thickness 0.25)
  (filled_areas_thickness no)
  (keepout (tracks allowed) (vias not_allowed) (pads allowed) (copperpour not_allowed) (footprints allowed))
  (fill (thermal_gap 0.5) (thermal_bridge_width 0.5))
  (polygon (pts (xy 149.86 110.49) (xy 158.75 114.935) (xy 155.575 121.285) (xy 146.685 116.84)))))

